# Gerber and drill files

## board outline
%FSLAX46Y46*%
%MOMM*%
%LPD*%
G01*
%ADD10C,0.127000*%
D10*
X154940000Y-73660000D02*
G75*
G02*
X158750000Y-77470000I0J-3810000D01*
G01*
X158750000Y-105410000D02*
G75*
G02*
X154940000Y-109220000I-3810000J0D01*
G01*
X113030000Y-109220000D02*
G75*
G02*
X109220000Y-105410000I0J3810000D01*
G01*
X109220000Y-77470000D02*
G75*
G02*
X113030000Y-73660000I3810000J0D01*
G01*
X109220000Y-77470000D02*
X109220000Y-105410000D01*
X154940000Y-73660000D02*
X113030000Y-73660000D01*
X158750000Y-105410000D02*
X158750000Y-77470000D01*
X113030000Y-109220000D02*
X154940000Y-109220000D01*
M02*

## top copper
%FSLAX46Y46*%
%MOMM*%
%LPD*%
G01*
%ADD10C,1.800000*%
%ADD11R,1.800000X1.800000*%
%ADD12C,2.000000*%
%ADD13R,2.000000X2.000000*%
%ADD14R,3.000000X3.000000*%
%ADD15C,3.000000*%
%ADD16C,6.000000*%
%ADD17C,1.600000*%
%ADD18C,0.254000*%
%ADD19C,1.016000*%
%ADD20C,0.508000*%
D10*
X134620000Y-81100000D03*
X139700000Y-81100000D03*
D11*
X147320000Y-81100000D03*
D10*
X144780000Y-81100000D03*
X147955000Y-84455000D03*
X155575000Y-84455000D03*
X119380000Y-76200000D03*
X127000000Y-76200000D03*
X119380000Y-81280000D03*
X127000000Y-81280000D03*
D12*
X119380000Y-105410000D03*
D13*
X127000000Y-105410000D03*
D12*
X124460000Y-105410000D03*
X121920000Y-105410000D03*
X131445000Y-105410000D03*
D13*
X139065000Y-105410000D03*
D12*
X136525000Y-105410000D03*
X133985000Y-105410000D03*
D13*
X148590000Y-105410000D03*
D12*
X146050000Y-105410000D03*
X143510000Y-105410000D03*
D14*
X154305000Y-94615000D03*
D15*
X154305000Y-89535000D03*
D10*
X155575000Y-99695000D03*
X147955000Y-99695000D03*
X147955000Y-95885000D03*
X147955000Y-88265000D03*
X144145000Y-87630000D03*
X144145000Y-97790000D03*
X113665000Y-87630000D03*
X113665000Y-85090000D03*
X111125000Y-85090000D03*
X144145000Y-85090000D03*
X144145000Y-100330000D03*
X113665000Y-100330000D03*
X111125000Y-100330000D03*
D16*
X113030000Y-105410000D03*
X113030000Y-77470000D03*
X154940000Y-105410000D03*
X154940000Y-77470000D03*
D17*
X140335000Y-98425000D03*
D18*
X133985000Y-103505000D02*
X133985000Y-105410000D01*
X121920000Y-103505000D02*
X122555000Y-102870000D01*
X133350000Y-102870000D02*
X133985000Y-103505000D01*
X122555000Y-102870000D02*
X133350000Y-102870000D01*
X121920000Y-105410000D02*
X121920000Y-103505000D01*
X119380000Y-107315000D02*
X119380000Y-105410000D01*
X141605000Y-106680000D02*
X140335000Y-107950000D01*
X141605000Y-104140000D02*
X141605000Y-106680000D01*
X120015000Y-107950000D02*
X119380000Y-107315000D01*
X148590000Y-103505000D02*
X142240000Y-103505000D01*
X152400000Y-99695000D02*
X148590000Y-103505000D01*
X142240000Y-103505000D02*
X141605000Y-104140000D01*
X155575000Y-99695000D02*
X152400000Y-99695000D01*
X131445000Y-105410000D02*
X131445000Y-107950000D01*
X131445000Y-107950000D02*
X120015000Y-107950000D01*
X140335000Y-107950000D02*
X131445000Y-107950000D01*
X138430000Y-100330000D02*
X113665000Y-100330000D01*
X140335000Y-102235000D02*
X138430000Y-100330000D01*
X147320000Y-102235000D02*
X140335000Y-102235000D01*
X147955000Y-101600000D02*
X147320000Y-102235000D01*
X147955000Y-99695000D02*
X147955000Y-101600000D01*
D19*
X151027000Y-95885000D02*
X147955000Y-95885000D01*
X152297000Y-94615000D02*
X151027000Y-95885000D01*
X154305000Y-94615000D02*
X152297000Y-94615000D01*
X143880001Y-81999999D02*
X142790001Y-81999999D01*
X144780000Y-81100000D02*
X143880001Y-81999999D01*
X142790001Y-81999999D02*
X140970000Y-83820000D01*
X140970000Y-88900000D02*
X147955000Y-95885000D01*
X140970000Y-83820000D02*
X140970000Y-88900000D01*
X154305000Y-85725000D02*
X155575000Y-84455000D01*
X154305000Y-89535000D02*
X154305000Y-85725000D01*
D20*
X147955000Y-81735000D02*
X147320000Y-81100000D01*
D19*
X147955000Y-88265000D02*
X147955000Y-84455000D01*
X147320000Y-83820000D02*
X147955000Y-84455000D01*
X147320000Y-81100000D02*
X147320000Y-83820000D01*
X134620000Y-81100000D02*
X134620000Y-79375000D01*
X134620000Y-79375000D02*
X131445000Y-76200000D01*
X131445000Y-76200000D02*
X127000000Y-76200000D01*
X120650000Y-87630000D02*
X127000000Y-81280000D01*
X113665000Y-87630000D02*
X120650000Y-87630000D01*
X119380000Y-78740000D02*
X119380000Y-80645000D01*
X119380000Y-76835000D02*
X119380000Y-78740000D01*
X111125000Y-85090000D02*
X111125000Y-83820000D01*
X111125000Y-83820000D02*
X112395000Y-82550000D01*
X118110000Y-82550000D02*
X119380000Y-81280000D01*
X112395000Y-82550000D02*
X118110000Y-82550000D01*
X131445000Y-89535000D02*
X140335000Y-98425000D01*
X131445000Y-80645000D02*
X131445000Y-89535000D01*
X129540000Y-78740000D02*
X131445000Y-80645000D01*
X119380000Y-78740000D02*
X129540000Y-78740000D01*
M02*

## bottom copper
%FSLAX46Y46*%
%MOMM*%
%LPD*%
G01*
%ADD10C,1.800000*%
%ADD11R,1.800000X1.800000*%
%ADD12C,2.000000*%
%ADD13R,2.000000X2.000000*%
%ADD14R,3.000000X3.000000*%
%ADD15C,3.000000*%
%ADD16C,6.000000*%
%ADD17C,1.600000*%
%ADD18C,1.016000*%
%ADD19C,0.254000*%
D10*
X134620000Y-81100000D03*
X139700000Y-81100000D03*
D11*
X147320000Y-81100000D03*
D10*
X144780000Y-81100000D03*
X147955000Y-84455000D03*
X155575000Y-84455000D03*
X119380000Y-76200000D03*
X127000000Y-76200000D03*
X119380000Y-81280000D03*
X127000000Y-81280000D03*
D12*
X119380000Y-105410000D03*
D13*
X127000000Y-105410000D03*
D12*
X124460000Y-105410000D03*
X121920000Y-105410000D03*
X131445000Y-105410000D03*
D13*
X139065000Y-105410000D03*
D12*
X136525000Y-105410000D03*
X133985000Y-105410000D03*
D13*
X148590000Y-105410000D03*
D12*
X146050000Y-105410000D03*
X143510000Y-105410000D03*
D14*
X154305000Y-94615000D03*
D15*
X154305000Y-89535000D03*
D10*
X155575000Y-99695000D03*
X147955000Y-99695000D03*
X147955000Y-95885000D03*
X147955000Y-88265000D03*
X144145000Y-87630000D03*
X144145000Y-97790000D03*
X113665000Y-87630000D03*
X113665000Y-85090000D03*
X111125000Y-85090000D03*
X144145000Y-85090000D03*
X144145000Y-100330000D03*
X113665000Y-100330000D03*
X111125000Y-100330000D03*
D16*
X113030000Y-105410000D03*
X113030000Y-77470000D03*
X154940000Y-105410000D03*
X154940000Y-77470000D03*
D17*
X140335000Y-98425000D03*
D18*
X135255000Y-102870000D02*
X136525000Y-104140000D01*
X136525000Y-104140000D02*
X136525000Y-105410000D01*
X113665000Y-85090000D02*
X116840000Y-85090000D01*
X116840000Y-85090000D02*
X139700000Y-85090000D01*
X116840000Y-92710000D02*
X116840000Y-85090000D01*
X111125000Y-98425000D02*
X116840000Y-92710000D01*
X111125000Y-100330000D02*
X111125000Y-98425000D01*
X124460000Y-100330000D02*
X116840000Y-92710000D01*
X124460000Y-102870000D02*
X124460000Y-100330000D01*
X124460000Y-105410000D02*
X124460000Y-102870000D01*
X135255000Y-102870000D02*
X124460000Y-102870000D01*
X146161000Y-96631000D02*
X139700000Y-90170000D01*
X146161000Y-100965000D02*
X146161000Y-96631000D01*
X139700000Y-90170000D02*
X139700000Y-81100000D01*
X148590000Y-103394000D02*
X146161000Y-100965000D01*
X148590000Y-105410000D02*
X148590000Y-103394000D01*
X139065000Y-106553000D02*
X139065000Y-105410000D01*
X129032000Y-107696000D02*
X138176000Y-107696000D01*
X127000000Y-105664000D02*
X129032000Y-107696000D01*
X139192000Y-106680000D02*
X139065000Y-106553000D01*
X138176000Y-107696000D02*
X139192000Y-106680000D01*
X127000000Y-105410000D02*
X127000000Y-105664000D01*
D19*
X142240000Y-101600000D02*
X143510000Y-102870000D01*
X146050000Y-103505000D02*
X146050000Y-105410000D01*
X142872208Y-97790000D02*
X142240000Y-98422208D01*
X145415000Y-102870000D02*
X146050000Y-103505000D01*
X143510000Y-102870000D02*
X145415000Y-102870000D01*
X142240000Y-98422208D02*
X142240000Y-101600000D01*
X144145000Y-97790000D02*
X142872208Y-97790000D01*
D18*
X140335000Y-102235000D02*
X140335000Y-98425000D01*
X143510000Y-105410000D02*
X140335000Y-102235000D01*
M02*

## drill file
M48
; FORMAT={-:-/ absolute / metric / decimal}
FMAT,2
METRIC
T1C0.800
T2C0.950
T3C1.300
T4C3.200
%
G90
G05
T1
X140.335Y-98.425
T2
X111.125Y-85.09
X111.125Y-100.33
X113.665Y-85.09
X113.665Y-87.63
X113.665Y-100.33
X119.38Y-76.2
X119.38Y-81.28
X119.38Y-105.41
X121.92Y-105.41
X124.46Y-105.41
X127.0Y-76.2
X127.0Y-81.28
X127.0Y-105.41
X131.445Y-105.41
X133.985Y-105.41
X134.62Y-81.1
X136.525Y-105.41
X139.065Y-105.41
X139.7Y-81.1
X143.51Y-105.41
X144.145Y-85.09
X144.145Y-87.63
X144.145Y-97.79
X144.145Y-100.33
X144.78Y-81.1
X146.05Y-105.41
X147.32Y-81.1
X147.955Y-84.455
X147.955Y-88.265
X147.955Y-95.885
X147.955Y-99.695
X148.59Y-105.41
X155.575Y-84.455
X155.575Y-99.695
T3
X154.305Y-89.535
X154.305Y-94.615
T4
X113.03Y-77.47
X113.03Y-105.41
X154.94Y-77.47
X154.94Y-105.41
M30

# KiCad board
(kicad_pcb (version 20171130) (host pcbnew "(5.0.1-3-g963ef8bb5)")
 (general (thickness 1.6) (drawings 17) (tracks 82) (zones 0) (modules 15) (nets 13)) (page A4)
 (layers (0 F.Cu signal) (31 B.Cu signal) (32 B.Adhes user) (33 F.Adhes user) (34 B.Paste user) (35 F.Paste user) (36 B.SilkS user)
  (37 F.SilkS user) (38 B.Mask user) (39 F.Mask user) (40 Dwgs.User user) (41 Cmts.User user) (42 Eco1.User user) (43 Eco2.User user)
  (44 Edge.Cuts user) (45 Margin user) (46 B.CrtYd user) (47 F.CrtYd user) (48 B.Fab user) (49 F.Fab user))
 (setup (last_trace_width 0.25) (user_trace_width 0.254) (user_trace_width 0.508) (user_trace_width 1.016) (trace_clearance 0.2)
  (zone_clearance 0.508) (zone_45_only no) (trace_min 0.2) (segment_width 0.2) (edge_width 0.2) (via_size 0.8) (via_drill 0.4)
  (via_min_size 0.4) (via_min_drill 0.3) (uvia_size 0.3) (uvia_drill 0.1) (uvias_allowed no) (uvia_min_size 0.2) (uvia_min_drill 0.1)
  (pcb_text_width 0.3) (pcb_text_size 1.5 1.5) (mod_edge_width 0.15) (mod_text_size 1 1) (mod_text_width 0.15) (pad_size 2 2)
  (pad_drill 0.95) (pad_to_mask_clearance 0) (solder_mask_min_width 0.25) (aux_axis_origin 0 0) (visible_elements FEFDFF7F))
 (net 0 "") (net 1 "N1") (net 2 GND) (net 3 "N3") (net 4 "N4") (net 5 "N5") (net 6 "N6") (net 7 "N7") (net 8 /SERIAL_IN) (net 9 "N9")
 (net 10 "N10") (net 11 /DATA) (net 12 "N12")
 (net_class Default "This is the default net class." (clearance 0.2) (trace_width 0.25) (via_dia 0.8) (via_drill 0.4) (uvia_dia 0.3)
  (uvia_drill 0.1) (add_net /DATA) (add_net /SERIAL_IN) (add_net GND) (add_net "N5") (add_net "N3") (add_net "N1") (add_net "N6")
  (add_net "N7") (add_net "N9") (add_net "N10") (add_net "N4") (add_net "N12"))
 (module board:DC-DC (layer F.Cu) (at 147.32 76.2 180)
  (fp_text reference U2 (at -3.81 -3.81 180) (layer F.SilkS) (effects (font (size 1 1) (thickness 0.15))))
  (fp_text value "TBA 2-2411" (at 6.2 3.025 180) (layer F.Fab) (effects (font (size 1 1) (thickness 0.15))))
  (pad 4 thru_hole circle (at 12.7 -4.9 180) (size 1.8 1.8) (drill 0.95) (layers *.Cu *.Mask) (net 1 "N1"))
  (pad 3 thru_hole circle (at 7.62 -4.9 180) (size 1.8 1.8) (drill 0.95) (layers *.Cu *.Mask) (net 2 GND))
  (pad 1 thru_hole rect (at 0 -4.9 180) (size 1.8 1.8) (drill 0.95) (layers *.Cu *.Mask) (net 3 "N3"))
  (pad 2 thru_hole circle (at 2.54 -4.9 180) (size 1.8 1.8) (drill 0.95) (layers *.Cu *.Mask) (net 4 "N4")))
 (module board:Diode (layer F.Cu) (at 147.955 84.455)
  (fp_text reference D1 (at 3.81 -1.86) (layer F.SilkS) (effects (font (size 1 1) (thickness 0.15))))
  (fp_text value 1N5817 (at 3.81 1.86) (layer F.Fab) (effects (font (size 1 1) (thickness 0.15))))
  (pad K thru_hole circle (at 0 0) (size 1.8 1.8) (drill 0.95) (layers *.Cu *.Mask) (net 3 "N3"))
  (pad A thru_hole circle (at 7.62 0) (size 1.8 1.8) (drill 0.95) (layers *.Cu *.Mask) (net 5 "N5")))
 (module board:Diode (layer F.Cu) (at 119.38 76.2)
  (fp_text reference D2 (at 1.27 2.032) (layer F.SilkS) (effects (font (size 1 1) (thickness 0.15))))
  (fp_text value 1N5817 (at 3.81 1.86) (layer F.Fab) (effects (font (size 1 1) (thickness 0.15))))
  (pad K thru_hole circle (at 0 0) (size 1.8 1.8) (drill 0.95) (layers *.Cu *.Mask) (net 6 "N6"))
  (pad A thru_hole circle (at 7.62 0) (size 1.8 1.8) (drill 0.95) (layers *.Cu *.Mask) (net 1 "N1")))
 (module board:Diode (layer F.Cu) (at 119.38 81.28)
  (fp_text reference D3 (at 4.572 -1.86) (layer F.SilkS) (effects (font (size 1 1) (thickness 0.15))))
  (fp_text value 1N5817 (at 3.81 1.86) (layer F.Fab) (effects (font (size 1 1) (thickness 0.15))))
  (pad K thru_hole circle (at 0 0) (size 1.8 1.8) (drill 0.95) (layers *.Cu *.Mask) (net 6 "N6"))
  (pad A thru_hole circle (at 7.62 0) (size 1.8 1.8) (drill 0.95) (layers *.Cu *.Mask) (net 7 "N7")))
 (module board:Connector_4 (layer F.Cu) (at 127 105.41 270)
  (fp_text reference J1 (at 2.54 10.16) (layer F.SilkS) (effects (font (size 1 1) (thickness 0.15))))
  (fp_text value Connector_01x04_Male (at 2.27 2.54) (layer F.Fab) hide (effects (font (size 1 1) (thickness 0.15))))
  (pad 4 thru_hole circle (at 0 7.62 270) (size 2 2) (drill 0.95) (layers *.Cu *.Mask) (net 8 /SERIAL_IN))
  (pad 1 thru_hole rect (at 0 0 270) (size 2 2) (drill 0.95) (layers *.Cu *.Mask) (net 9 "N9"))
  (pad 2 thru_hole circle (at 0 2.54 270) (size 2 2) (drill 0.95) (layers *.Cu *.Mask) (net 2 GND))
  (pad 3 thru_hole circle (at 0 5.08 270) (size 2 2) (drill 0.95) (layers *.Cu *.Mask) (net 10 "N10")))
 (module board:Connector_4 (layer F.Cu) (at 139.065 105.41 270)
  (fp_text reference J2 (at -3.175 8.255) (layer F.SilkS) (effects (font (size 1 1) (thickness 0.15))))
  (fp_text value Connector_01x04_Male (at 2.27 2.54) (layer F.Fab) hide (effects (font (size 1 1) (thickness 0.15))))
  (pad 4 thru_hole circle (at 0 7.62 270) (size 2 2) (drill 0.95) (layers *.Cu *.Mask) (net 8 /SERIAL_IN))
  (pad 1 thru_hole rect (at 0 0 270) (size 2 2) (drill 0.95) (layers *.Cu *.Mask) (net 9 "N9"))
  (pad 2 thru_hole circle (at 0 2.54 270) (size 2 2) (drill 0.95) (layers *.Cu *.Mask) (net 2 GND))
  (pad 3 thru_hole circle (at 0 5.08 270) (size 2 2) (drill 0.95) (layers *.Cu *.Mask) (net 10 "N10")))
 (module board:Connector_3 (layer F.Cu) (at 148.59 105.41 270)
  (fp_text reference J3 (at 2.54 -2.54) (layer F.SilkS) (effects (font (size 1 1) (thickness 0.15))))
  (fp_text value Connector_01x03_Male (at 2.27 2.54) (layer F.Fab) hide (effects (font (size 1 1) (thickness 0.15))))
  (pad 1 thru_hole rect (at 0 0 270) (size 2 2) (drill 0.95) (layers *.Cu *.Mask) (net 2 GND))
  (pad 2 thru_hole circle (at 0 2.54 270) (size 2 2) (drill 0.95) (layers *.Cu *.Mask) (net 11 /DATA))
  (pad 3 thru_hole circle (at 0 5.08 270) (size 2 2) (drill 0.95) (layers *.Cu *.Mask) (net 6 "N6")))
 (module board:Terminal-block (layer F.Cu) (at 154.305 94.615 90)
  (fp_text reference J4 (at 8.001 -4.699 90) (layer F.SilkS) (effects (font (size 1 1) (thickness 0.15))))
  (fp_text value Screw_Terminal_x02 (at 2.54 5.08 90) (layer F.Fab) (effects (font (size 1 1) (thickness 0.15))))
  (pad 1 thru_hole rect (at 0 0 90) (size 3 3) (drill 1.3) (layers *.Cu *.Mask) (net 4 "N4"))
  (pad 2 thru_hole circle (at 5.08 0 90) (size 3 3) (drill 1.3) (layers *.Cu *.Mask) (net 5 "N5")))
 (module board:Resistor (layer F.Cu) (at 155.575 99.695 180)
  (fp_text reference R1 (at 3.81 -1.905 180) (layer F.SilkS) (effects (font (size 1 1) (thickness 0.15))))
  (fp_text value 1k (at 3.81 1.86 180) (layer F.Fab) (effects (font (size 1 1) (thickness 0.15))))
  (pad 1 thru_hole circle (at 0 0 180) (size 1.8 1.8) (drill 0.95) (layers *.Cu *.Mask) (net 8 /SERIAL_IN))
  (pad 2 thru_hole circle (at 7.62 0 180) (size 1.8 1.8) (drill 0.95) (layers *.Cu *.Mask) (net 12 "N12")))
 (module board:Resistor (layer F.Cu) (at 147.955 95.885 90)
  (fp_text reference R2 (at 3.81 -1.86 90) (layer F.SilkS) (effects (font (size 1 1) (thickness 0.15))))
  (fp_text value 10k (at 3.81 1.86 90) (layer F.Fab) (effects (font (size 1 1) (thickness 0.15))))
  (pad 1 thru_hole circle (at 0 0 90) (size 1.8 1.8) (drill 0.95) (layers *.Cu *.Mask) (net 4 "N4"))
  (pad 2 thru_hole circle (at 7.62 0 90) (size 1.8 1.8) (drill 0.95) (layers *.Cu *.Mask) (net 3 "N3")))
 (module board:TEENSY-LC (layer F.Cu) (at 111.125 100.33)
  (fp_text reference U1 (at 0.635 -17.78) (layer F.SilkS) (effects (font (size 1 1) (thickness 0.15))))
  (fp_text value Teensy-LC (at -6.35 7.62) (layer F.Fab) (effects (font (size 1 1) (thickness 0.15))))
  (pad 19 thru_hole circle (at 33.02 -12.7) (size 1.8 1.8) (drill 0.95) (layers *.Cu *.Mask))
  (pad 15 thru_hole circle (at 33.02 -2.54) (size 1.8 1.8) (drill 0.95) (layers *.Cu *.Mask) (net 11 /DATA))
  (pad 34 thru_hole circle (at 2.54 -12.7) (size 1.8 1.8) (drill 0.95) (layers *.Cu *.Mask) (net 7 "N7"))
  (pad 32 thru_hole circle (at 2.54 -15.24) (size 1.8 1.8) (drill 0.95) (layers *.Cu *.Mask) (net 2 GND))
  (pad 33 thru_hole circle (at 0 -15.24) (size 1.8 1.8) (drill 0.95) (layers *.Cu *.Mask) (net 6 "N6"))
  (pad 20 thru_hole circle (at 33.02 -15.24) (size 1.8 1.8) (drill 0.95) (layers *.Cu *.Mask))
  (pad 14 thru_hole circle (at 33.02 0) (size 1.8 1.8) (drill 0.95) (layers *.Cu *.Mask))
  (pad 2 thru_hole circle (at 2.54 0) (size 1.8 1.8) (drill 0.95) (layers *.Cu *.Mask) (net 12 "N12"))
  (pad 1 thru_hole circle (at 0 0) (size 1.8 1.8) (drill 0.95) (layers *.Cu *.Mask) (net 2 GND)))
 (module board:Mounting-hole (layer F.Cu) (at 113.03 105.41)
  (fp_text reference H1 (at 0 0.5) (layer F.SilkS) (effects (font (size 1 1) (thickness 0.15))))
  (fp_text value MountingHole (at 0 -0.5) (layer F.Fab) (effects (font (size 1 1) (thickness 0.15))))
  (pad 1 thru_hole circle (at 0 0) (size 6 6) (drill 3.2) (layers *.Cu *.Mask)))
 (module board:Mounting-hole (layer F.Cu) (at 113.03 77.47)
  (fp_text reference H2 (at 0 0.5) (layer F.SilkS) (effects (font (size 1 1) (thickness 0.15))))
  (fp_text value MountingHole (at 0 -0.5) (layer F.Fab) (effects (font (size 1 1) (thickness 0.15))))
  (pad 1 thru_hole circle (at 0 0) (size 6 6) (drill 3.2) (layers *.Cu *.Mask)))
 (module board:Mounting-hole (layer F.Cu) (at 154.94 105.41)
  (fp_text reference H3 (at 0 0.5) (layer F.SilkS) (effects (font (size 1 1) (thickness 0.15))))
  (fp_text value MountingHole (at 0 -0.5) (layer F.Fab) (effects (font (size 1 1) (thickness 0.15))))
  (pad 1 thru_hole circle (at 0 0) (size 6 6) (drill 3.2) (layers *.Cu *.Mask)))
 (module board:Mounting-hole (layer F.Cu) (at 154.94 77.47)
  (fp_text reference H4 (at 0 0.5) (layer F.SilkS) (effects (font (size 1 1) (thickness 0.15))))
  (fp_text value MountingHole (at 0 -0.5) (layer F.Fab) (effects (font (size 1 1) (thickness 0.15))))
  (pad 1 thru_hole circle (at 0 0) (size 6 6) (drill 3.2) (layers *.Cu *.Mask)))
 (gr_arc (start 154.94 77.47) (end 158.75 77.47) (angle -90) (layer Edge.Cuts) (width 0.127))
 (gr_arc (start 154.94 105.41) (end 154.94 109.22) (angle -90) (layer Edge.Cuts) (width 0.127))
 (gr_arc (start 113.03 105.41) (end 109.22 105.41) (angle -90) (layer Edge.Cuts) (width 0.127))
 (gr_arc (start 113.03 77.47) (end 113.03 73.66) (angle -90) (layer Edge.Cuts) (width 0.127))
 (gr_line (start 109.22 77.47) (end 109.22 105.41) (layer Edge.Cuts) (width 0.127))
 (gr_line (start 154.94 73.66) (end 113.03 73.66) (layer Edge.Cuts) (width 0.127))
 (gr_line (start 158.75 105.41) (end 158.75 77.47) (layer Edge.Cuts) (width 0.127))
 (gr_line (start 113.03 109.22) (end 154.94 109.22) (layer Edge.Cuts) (width 0.127))
 (segment (start 133.985 103.505) (end 133.985 105.41) (width 0.254) (layer F.Cu) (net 10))
 (segment (start 121.92 103.505) (end 122.555 102.87) (width 0.254) (layer F.Cu) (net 10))
 (segment (start 133.35 102.87) (end 133.985 103.505) (width 0.254) (layer F.Cu) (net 10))
 (segment (start 122.555 102.87) (end 133.35 102.87) (width 0.254) (layer F.Cu) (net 10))
 (segment (start 121.92 105.41) (end 121.92 103.505) (width 0.254) (layer F.Cu) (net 10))
 (segment (start 135.255 102.87) (end 136.525 104.14) (width 1.016) (layer B.Cu) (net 2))
 (segment (start 136.525 104.14) (end 136.525 105.41) (width 1.016) (layer B.Cu) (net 2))
 (segment (start 113.665 85.09) (end 116.84 85.09) (width 1.016) (layer B.Cu) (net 2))
 (segment (start 116.84 85.09) (end 139.7 85.09) (width 1.016) (layer B.Cu) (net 2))
 (segment (start 116.84 92.71) (end 116.84 85.09) (width 1.016) (layer B.Cu) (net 2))
 (segment (start 111.125 98.425) (end 116.84 92.71) (width 1.016) (layer B.Cu) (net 2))
 (segment (start 111.125 100.33) (end 111.125 98.425) (width 1.016) (layer B.Cu) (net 2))
 (segment (start 124.46 100.33) (end 116.84 92.71) (width 1.016) (layer B.Cu) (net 2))
 (segment (start 124.46 102.87) (end 124.46 100.33) (width 1.016) (layer B.Cu) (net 2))
 (segment (start 124.46 105.41) (end 124.46 102.87) (width 1.016) (layer B.Cu) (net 2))
 (segment (start 135.255 102.87) (end 124.46 102.87) (width 1.016) (layer B.Cu) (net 2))
 (segment (start 146.161 96.631) (end 139.7 90.17) (width 1.016) (layer B.Cu) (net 2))
 (segment (start 146.161 100.965) (end 146.161 96.631) (width 1.016) (layer B.Cu) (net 2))
 (segment (start 139.7 90.17) (end 139.7 81.1) (width 1.016) (layer B.Cu) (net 2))
 (segment (start 148.59 103.394) (end 146.161 100.965) (width 1.016) (layer B.Cu) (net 2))
 (segment (start 148.59 105.41) (end 148.59 103.394) (width 1.016) (layer B.Cu) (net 2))
 (segment (start 139.065 106.553) (end 139.065 105.41) (width 1.016) (layer B.Cu) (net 9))
 (segment (start 129.032 107.696) (end 138.176 107.696) (width 1.016) (layer B.Cu) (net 9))
 (segment (start 127 105.664) (end 129.032 107.696) (width 1.016) (layer B.Cu) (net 9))
 (segment (start 139.192 106.68) (end 139.065 106.553) (width 1.016) (layer B.Cu) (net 9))
 (segment (start 138.176 107.696) (end 139.192 106.68) (width 1.016) (layer B.Cu) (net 9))
 (segment (start 127 105.41) (end 127 105.664) (width 1.016) (layer B.Cu) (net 9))
 (segment (start 119.38 107.315) (end 119.38 105.41) (width 0.254) (layer F.Cu) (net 8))
 (segment (start 141.605 106.68) (end 140.335 107.95) (width 0.254) (layer F.Cu) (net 8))
 (segment (start 141.605 104.14) (end 141.605 106.68) (width 0.254) (layer F.Cu) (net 8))
 (segment (start 120.015 107.95) (end 119.38 107.315) (width 0.254) (layer F.Cu) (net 8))
 (segment (start 148.59 103.505) (end 142.24 103.505) (width 0.254) (layer F.Cu) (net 8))
 (segment (start 152.4 99.695) (end 148.59 103.505) (width 0.254) (layer F.Cu) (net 8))
 (segment (start 142.24 103.505) (end 141.605 104.14) (width 0.254) (layer F.Cu) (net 8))
 (segment (start 155.575 99.695) (end 152.4 99.695) (width 0.254) (layer F.Cu) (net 8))
 (segment (start 131.445 105.41) (end 131.445 107.95) (width 0.254) (layer F.Cu) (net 8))
 (segment (start 131.445 107.95) (end 120.015 107.95) (width 0.254) (layer F.Cu) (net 8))
 (segment (start 140.335 107.95) (end 131.445 107.95) (width 0.254) (layer F.Cu) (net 8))
 (segment (start 142.24 101.6) (end 143.51 102.87) (width 0.254) (layer B.Cu) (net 11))
 (segment (start 146.05 103.505) (end 146.05 105.41) (width 0.254) (layer B.Cu) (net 11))
 (segment (start 142.872208 97.79) (end 142.24 98.422208) (width 0.254) (layer B.Cu) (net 11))
 (segment (start 145.415 102.87) (end 146.05 103.505) (width 0.254) (layer B.Cu) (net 11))
 (segment (start 143.51 102.87) (end 145.415 102.87) (width 0.254) (layer B.Cu) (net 11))
 (segment (start 142.24 98.422208) (end 142.24 101.6) (width 0.254) (layer B.Cu) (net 11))
 (segment (start 144.145 97.79) (end 142.872208 97.79) (width 0.254) (layer B.Cu) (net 11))
 (segment (start 138.43 100.33) (end 113.665 100.33) (width 0.254) (layer F.Cu) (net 12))
 (segment (start 140.335 102.235) (end 138.43 100.33) (width 0.254) (layer F.Cu) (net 12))
 (segment (start 147.32 102.235) (end 140.335 102.235) (width 0.254) (layer F.Cu) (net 12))
 (segment (start 147.955 101.6) (end 147.32 102.235) (width 0.254) (layer F.Cu) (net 12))
 (segment (start 147.955 99.695) (end 147.955 101.6) (width 0.254) (layer F.Cu) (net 12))
 (segment (start 151.027 95.885) (end 147.955 95.885) (width 1.016) (layer F.Cu) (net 4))
 (segment (start 152.297 94.615) (end 151.027 95.885) (width 1.016) (layer F.Cu) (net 4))
 (segment (start 154.305 94.615) (end 152.297 94.615) (width 1.016) (layer F.Cu) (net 4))
 (segment (start 143.880001 81.999999) (end 142.790001 81.999999) (width 1.016) (layer F.Cu) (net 4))
 (segment (start 144.78 81.1) (end 143.880001 81.999999) (width 1.016) (layer F.Cu) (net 4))
 (segment (start 142.790001 81.999999) (end 140.97 83.82) (width 1.016) (layer F.Cu) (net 4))
 (segment (start 140.97 88.9) (end 147.955 95.885) (width 1.016) (layer F.Cu) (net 4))
 (segment (start 140.97 83.82) (end 140.97 88.9) (width 1.016) (layer F.Cu) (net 4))
 (segment (start 154.305 85.725) (end 155.575 84.455) (width 1.016) (layer F.Cu) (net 5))
 (segment (start 154.305 89.535) (end 154.305 85.725) (width 1.016) (layer F.Cu) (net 5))
 (segment (start 147.955 81.735) (end 147.32 81.1) (width 0.508) (layer F.Cu) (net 3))
 (segment (start 147.955 88.265) (end 147.955 84.455) (width 1.016) (layer F.Cu) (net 3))
 (segment (start 147.32 83.82) (end 147.955 84.455) (width 1.016) (layer F.Cu) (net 3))
 (segment (start 147.32 81.1) (end 147.32 83.82) (width 1.016) (layer F.Cu) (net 3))
 (segment (start 134.62 81.1) (end 134.62 79.375) (width 1.016) (layer F.Cu) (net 1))
 (segment (start 134.62 79.375) (end 131.445 76.2) (width 1.016) (layer F.Cu) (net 1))
 (segment (start 131.445 76.2) (end 127 76.2) (width 1.016) (layer F.Cu) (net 1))
 (segment (start 120.65 87.63) (end 127 81.28) (width 1.016) (layer F.Cu) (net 7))
 (segment (start 113.665 87.63) (end 120.65 87.63) (width 1.016) (layer F.Cu) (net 7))
 (via (at 140.335 98.425) (size 1.6) (drill 0.8) (layers F.Cu B.Cu) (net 6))
 (segment (start 119.38 78.74) (end 119.38 80.645) (width 1.016) (layer F.Cu) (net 6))
 (segment (start 119.38 76.835) (end 119.38 78.74) (width 1.016) (layer F.Cu) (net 6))
 (segment (start 111.125 85.09) (end 111.125 83.82) (width 1.016) (layer F.Cu) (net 6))
 (segment (start 111.125 83.82) (end 112.395 82.55) (width 1.016) (layer F.Cu) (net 6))
 (segment (start 118.11 82.55) (end 119.38 81.28) (width 1.016) (layer F.Cu) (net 6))
 (segment (start 112.395 82.55) (end 118.11 82.55) (width 1.016) (layer F.Cu) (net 6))
 (segment (start 140.335 102.235) (end 140.335 98.425) (width 1.016) (layer B.Cu) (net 6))
 (segment (start 143.51 105.41) (end 140.335 102.235) (width 1.016) (layer B.Cu) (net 6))
 (segment (start 131.445 89.535) (end 140.335 98.425) (width 1.016) (layer F.Cu) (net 6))
 (segment (start 131.445 80.645) (end 131.445 89.535) (width 1.016) (layer F.Cu) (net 6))
 (segment (start 129.54 78.74) (end 131.445 80.645) (width 1.016) (layer F.Cu) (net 6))
 (segment (start 119.38 78.74) (end 129.54 78.74) (width 1.016) (layer F.Cu) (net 6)))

